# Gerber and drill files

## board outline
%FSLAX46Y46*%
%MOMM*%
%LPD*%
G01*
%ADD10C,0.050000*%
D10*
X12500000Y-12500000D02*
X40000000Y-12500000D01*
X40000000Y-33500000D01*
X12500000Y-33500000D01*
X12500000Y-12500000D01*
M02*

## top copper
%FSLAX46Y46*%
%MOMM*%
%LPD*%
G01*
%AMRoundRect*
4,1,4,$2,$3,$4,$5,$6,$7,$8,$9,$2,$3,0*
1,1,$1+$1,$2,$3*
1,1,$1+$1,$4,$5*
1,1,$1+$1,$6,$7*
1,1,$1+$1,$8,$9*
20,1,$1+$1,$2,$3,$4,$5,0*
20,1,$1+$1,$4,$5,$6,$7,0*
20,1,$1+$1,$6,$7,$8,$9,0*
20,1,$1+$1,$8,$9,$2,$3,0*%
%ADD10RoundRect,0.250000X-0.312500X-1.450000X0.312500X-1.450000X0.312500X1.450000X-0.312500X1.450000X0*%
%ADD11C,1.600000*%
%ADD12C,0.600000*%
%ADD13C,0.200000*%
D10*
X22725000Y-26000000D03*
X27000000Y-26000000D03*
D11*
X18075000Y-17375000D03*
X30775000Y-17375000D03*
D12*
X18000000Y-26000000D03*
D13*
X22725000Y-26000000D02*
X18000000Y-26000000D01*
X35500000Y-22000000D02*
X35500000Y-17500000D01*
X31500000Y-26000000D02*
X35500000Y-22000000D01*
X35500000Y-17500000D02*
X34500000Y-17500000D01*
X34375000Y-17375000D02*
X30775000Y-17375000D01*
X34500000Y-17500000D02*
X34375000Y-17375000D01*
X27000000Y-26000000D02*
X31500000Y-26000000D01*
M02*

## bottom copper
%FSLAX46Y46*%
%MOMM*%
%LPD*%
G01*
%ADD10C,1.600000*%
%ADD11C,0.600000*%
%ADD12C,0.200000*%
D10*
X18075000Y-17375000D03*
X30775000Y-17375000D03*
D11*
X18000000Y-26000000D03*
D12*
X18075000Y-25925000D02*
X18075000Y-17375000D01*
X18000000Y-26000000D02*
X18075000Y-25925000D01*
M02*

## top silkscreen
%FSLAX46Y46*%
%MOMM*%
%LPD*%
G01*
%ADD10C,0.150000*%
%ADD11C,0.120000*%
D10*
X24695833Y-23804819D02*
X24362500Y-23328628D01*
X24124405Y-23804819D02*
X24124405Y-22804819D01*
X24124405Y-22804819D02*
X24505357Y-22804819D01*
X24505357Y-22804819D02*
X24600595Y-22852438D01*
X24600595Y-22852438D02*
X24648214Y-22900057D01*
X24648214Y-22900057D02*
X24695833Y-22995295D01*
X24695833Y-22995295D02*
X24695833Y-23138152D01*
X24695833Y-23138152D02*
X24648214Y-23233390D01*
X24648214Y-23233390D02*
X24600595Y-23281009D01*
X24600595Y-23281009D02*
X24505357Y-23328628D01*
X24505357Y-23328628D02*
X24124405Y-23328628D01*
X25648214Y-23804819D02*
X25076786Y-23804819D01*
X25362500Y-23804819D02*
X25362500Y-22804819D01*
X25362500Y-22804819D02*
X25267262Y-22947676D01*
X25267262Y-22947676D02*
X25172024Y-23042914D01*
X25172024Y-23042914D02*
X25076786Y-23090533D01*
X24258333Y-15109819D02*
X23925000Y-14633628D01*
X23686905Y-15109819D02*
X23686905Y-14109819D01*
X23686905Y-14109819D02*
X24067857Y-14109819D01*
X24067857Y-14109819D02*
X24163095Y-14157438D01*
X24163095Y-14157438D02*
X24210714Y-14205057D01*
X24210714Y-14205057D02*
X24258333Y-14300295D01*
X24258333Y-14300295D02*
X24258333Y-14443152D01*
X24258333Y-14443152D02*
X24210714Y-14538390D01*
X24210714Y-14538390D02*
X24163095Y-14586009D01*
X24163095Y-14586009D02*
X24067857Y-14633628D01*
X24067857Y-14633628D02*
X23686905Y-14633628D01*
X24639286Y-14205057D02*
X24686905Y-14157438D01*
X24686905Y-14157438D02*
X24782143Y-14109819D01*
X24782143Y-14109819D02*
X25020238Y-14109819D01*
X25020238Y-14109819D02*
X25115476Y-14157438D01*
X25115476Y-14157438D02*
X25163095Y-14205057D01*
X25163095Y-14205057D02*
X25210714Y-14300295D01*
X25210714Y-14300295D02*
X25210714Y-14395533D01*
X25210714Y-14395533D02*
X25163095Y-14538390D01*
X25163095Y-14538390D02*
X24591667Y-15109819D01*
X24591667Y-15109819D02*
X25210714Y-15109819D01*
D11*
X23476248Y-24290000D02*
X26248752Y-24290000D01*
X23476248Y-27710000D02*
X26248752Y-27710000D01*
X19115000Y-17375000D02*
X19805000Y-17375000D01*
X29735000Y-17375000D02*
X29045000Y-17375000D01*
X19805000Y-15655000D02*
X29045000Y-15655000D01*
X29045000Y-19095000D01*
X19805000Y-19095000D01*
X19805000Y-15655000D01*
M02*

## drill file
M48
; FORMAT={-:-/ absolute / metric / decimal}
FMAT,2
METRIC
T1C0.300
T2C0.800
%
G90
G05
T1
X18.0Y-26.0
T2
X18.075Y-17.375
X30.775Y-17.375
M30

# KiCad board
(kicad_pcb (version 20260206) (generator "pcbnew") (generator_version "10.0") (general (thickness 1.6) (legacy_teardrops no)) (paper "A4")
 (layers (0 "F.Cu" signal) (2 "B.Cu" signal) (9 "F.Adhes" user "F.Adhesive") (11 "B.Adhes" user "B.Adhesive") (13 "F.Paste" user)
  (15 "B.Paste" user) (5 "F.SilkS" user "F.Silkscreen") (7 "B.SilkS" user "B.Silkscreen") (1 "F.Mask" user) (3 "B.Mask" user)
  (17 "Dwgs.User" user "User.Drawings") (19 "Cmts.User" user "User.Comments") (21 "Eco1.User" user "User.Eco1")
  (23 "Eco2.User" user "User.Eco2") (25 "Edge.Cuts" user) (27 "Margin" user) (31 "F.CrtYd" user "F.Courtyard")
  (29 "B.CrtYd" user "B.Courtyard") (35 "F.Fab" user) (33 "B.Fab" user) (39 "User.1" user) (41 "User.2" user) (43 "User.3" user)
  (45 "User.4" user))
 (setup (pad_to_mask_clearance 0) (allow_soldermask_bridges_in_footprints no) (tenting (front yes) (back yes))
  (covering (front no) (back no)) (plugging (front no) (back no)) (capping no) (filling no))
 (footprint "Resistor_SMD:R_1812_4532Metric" (layer "F.Cu") (at 24.8625 26)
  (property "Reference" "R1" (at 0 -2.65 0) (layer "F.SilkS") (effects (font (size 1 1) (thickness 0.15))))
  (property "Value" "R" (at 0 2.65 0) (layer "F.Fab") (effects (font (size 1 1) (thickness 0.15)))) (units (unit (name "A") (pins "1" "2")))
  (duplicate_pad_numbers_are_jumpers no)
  (fp_line (start -1.386252 -1.71) (end 1.386252 -1.71) (stroke (width 0.12) (type solid)) (layer "F.SilkS"))
  (fp_line (start -1.386252 1.71) (end 1.386252 1.71) (stroke (width 0.12) (type solid)) (layer "F.SilkS"))
  (pad "1" smd roundrect (at -2.1375 0) (size 1.125 3.4) (layers "F.Cu" "F.Mask" "F.Paste") (roundrect_rratio 0.222222)
   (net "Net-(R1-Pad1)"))
  (pad "2" smd roundrect (at 2.1375 0) (size 1.125 3.4) (layers "F.Cu" "F.Mask" "F.Paste") (roundrect_rratio 0.222222) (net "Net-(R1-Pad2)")))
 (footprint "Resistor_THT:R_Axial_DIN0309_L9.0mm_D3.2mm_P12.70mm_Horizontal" (layer "F.Cu") (at 18.075 17.375)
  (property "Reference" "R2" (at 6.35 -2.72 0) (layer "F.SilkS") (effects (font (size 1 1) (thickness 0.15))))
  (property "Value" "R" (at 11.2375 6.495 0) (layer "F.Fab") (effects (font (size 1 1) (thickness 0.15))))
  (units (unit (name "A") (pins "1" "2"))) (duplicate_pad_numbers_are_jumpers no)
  (fp_line (start 1.04 0) (end 1.73 0) (stroke (width 0.12) (type solid)) (layer "F.SilkS"))
  (fp_line (start 11.66 0) (end 10.97 0) (stroke (width 0.12) (type solid)) (layer "F.SilkS"))
  (fp_rect (start 1.73 -1.72) (end 10.97 1.72) (stroke (width 0.12) (type solid)) (fill no) (layer "F.SilkS"))
  (pad "1" thru_hole circle (at 0 0) (size 1.6 1.6) (drill 0.8) (layers "*.Cu" "*.Mask") (remove_unused_layers no) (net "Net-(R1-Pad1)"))
  (pad "2" thru_hole circle (at 12.7 0) (size 1.6 1.6) (drill 0.8) (layers "*.Cu" "*.Mask") (remove_unused_layers no) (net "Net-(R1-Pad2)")))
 (gr_rect (start 12.5 12.5) (end 40 33.5) (stroke (width 0.05) (type default)) (fill no) (layer "Edge.Cuts"))
 (segment (start 22.725 26) (end 18 26) (width 0.2) (layer "F.Cu") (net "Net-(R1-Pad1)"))
 (via (at 18 26) (size 0.6) (drill 0.3) (layers "F.Cu" "B.Cu") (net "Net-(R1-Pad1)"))
 (segment (start 18.075 25.925) (end 18.075 17.375) (width 0.2) (layer "B.Cu") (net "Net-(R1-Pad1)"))
 (segment (start 18 26) (end 18.075 25.925) (width 0.2) (layer "B.Cu") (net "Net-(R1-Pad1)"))
 (segment (start 35.5 22) (end 35.5 17.5) (width 0.2) (layer "F.Cu") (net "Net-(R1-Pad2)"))
 (segment (start 31.5 26) (end 35.5 22) (width 0.2) (layer "F.Cu") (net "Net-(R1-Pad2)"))
 (segment (start 35.5 17.5) (end 34.5 17.5) (width 0.2) (layer "F.Cu") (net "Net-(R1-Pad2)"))
 (segment (start 34.375 17.375) (end 30.775 17.375) (width 0.2) (layer "F.Cu") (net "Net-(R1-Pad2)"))
 (segment (start 34.5 17.5) (end 34.375 17.375) (width 0.2) (layer "F.Cu") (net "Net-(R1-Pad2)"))
 (segment (start 27 26) (end 31.5 26) (width 0.2) (layer "F.Cu") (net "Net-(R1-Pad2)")))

